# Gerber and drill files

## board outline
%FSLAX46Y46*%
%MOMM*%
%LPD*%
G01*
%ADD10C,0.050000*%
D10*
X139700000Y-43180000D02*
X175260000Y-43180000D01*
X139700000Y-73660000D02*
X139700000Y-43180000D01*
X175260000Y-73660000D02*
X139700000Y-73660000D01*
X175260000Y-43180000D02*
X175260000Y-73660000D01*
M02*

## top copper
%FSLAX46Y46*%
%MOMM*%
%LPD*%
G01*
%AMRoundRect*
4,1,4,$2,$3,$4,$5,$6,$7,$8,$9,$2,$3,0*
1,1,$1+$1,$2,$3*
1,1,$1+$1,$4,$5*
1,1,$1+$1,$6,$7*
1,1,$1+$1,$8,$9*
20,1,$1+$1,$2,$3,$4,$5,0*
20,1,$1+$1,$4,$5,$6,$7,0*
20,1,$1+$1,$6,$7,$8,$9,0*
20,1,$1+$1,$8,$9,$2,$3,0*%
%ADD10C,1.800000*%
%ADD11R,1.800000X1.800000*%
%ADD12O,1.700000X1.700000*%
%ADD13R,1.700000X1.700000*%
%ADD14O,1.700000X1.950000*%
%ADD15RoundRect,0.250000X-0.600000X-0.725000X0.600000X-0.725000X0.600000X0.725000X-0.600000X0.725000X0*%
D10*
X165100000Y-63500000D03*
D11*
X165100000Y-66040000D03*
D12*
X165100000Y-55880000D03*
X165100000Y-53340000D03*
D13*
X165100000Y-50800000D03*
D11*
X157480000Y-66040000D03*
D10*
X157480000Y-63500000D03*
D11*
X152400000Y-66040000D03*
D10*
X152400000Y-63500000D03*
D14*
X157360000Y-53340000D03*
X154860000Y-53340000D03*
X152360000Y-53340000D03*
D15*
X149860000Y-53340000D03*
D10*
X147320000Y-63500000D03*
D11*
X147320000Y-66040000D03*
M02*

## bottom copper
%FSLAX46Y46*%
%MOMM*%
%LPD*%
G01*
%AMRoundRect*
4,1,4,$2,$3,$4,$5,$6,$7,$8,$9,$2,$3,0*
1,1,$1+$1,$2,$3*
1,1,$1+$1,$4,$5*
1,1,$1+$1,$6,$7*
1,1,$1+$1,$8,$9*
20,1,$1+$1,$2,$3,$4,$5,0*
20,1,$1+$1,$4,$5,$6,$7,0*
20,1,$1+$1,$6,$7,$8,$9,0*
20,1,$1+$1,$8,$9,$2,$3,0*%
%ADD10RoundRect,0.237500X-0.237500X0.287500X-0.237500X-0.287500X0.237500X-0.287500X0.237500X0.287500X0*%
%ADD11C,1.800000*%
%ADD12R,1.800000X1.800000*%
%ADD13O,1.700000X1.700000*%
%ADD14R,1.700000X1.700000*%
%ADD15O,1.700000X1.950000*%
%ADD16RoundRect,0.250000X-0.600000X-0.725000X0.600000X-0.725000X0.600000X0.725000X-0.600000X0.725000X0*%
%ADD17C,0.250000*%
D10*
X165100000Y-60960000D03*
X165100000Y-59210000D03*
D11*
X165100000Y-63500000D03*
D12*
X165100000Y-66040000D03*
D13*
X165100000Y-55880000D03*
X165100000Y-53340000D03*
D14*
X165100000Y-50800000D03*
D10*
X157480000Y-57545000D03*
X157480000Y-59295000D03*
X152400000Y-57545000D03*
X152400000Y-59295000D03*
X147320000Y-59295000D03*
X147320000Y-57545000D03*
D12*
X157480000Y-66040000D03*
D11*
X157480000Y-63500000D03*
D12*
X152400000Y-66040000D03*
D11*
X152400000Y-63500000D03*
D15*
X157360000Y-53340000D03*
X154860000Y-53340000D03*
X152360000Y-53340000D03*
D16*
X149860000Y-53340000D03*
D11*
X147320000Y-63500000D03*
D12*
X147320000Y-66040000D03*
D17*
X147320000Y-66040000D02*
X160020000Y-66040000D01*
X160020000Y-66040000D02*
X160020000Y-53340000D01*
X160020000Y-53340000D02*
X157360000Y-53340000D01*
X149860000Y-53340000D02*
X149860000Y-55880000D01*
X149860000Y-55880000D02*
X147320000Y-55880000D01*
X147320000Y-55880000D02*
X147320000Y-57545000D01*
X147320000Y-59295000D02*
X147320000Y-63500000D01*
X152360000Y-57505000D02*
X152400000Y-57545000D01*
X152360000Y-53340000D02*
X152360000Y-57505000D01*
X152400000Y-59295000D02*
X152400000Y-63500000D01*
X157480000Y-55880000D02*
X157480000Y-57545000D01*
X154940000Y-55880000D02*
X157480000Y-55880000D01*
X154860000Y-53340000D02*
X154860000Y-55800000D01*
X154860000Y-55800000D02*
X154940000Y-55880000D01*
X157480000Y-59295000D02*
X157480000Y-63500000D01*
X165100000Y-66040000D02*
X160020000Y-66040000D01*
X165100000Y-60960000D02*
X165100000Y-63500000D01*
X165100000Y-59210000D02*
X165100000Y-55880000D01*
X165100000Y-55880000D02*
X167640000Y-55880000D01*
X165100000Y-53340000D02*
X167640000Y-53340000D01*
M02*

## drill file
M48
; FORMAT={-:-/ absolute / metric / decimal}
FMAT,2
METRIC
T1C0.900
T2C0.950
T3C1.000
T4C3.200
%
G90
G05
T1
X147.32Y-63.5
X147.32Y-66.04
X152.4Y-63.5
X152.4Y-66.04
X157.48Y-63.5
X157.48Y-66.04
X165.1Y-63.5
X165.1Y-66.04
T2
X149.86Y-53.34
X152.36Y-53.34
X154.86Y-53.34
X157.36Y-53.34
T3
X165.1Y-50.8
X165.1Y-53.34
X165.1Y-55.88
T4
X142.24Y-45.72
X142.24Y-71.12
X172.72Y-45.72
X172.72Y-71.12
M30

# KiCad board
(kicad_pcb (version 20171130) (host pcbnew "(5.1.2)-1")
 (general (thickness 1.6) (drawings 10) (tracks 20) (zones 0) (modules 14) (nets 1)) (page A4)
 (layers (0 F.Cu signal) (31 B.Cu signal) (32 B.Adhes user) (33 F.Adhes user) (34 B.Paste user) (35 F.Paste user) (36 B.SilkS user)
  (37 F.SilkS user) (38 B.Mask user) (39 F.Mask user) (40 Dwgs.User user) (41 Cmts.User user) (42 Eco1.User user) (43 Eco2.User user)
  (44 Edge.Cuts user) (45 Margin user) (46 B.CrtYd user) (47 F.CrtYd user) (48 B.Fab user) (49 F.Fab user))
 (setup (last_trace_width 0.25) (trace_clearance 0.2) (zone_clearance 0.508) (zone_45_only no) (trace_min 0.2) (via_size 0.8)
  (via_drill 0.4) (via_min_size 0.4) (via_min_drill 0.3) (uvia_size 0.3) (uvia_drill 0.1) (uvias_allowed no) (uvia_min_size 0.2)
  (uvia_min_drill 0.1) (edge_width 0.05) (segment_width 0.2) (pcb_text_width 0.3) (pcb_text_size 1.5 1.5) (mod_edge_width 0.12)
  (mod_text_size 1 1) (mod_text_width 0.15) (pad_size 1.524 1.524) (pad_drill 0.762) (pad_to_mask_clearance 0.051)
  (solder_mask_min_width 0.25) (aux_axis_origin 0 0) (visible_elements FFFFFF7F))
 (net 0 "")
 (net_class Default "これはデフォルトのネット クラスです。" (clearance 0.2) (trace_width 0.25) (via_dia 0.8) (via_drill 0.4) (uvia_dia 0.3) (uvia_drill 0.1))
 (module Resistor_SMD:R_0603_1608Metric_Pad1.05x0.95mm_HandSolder (layer B.Cu) (at 165.1 60.085 270)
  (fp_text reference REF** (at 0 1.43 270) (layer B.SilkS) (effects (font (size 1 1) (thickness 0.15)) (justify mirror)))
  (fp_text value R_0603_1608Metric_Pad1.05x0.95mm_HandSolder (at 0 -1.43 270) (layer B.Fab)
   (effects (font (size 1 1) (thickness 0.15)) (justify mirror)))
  (pad 2 smd roundrect (at 0.875 0 270) (size 1.05 0.95) (layers B.Cu B.Paste B.Mask) (roundrect_rratio 0.25))
  (pad 1 smd roundrect (at -0.875 0 270) (size 1.05 0.95) (layers B.Cu B.Paste B.Mask) (roundrect_rratio 0.25)))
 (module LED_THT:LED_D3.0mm (layer F.Cu) (at 165.1 66.04 90)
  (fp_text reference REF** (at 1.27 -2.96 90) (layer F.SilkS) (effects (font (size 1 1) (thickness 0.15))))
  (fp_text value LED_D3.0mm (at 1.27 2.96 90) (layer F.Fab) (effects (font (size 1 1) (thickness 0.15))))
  (pad 2 thru_hole circle (at 2.54 0 90) (size 1.8 1.8) (drill 0.9) (layers *.Cu *.Mask))
  (pad 1 thru_hole rect (at 0 0 90) (size 1.8 1.8) (drill 0.9) (layers *.Cu *.Mask)))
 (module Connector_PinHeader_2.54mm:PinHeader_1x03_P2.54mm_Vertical (layer F.Cu) (at 165.1 50.8)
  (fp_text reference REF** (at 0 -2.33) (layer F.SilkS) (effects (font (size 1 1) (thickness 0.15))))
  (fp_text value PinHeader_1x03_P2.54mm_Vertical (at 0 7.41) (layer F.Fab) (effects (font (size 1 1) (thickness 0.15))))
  (pad 3 thru_hole oval (at 0 5.08) (size 1.7 1.7) (drill 1) (layers *.Cu *.Mask))
  (pad 2 thru_hole oval (at 0 2.54) (size 1.7 1.7) (drill 1) (layers *.Cu *.Mask))
  (pad 1 thru_hole rect (at 0 0) (size 1.7 1.7) (drill 1) (layers *.Cu *.Mask)))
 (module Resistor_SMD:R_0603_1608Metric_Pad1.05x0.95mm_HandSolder (layer B.Cu) (at 157.48 58.42 270)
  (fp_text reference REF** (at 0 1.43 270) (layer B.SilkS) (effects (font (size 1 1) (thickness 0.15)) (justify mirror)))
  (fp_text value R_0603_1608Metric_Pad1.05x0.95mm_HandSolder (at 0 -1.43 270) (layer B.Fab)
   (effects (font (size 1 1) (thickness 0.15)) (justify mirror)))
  (pad 1 smd roundrect (at -0.875 0 270) (size 1.05 0.95) (layers B.Cu B.Paste B.Mask) (roundrect_rratio 0.25))
  (pad 2 smd roundrect (at 0.875 0 270) (size 1.05 0.95) (layers B.Cu B.Paste B.Mask) (roundrect_rratio 0.25)))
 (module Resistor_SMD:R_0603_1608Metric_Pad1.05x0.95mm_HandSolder (layer B.Cu) (at 152.4 58.42 270)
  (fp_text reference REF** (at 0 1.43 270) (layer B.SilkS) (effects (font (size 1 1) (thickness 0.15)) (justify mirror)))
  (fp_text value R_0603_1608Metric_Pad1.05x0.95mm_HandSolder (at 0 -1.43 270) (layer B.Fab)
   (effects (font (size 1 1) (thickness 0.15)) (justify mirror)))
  (pad 1 smd roundrect (at -0.875 0 270) (size 1.05 0.95) (layers B.Cu B.Paste B.Mask) (roundrect_rratio 0.25))
  (pad 2 smd roundrect (at 0.875 0 270) (size 1.05 0.95) (layers B.Cu B.Paste B.Mask) (roundrect_rratio 0.25)))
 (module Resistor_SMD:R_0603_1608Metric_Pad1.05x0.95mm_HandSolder (layer B.Cu) (at 147.32 58.42 270)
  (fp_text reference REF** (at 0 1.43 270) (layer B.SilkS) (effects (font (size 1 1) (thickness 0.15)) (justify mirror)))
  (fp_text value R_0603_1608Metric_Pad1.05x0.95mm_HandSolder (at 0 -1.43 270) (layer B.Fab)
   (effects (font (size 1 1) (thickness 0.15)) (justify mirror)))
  (pad 2 smd roundrect (at 0.875 0 270) (size 1.05 0.95) (layers B.Cu B.Paste B.Mask) (roundrect_rratio 0.25))
  (pad 1 smd roundrect (at -0.875 0 270) (size 1.05 0.95) (layers B.Cu B.Paste B.Mask) (roundrect_rratio 0.25)))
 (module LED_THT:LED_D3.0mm (layer F.Cu) (at 157.48 66.04 90)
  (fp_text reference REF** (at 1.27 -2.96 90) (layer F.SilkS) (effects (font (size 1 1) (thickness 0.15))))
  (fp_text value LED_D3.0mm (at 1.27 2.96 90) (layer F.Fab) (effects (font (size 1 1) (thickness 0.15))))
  (pad 1 thru_hole rect (at 0 0 90) (size 1.8 1.8) (drill 0.9) (layers *.Cu *.Mask))
  (pad 2 thru_hole circle (at 2.54 0 90) (size 1.8 1.8) (drill 0.9) (layers *.Cu *.Mask)))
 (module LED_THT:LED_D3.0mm (layer F.Cu) (at 152.4 66.04 90)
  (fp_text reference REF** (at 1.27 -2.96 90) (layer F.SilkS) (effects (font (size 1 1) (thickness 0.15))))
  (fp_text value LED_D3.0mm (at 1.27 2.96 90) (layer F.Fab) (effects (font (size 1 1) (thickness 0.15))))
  (pad 1 thru_hole rect (at 0 0 90) (size 1.8 1.8) (drill 0.9) (layers *.Cu *.Mask))
  (pad 2 thru_hole circle (at 2.54 0 90) (size 1.8 1.8) (drill 0.9) (layers *.Cu *.Mask)))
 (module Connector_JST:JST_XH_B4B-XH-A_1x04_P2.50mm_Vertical (layer F.Cu) (at 149.86 53.34)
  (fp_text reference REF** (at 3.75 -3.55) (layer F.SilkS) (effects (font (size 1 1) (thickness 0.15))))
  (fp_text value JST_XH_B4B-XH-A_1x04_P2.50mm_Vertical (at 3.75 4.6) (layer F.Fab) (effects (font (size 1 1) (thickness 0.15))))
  (pad 4 thru_hole oval (at 7.5 0) (size 1.7 1.95) (drill 0.95) (layers *.Cu *.Mask))
  (pad 3 thru_hole oval (at 5 0) (size 1.7 1.95) (drill 0.95) (layers *.Cu *.Mask))
  (pad 2 thru_hole oval (at 2.5 0) (size 1.7 1.95) (drill 0.95) (layers *.Cu *.Mask))
  (pad 1 thru_hole roundrect (at 0 0) (size 1.7 1.95) (drill 0.95) (layers *.Cu *.Mask) (roundrect_rratio 0.147059)))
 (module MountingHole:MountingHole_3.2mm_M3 (layer F.Cu) (at 172.72 71.12)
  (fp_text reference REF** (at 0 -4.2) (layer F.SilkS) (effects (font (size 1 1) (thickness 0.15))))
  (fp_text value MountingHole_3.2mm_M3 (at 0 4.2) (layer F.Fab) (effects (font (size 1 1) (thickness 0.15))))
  (pad 1 np_thru_hole circle (at 0 0) (size 3.2 3.2) (drill 3.2) (layers *.Cu *.Mask)))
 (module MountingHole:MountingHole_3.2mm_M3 (layer F.Cu) (at 142.24 71.12)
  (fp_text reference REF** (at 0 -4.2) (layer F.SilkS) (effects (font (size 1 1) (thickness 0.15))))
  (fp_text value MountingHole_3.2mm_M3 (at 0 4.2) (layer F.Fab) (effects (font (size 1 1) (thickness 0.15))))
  (pad 1 np_thru_hole circle (at 0 0) (size 3.2 3.2) (drill 3.2) (layers *.Cu *.Mask)))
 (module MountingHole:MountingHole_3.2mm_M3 (layer F.Cu) (at 172.72 45.72)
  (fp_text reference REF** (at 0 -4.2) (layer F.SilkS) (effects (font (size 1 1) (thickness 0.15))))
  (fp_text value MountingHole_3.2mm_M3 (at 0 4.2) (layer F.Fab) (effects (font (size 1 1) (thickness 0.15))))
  (pad 1 np_thru_hole circle (at 0 0) (size 3.2 3.2) (drill 3.2) (layers *.Cu *.Mask)))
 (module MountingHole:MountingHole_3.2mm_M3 (layer F.Cu) (at 142.24 45.72)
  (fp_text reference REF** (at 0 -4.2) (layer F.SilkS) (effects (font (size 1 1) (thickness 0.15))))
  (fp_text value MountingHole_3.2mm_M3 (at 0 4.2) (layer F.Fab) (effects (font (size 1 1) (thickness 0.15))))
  (pad 1 np_thru_hole circle (at 0 0) (size 3.2 3.2) (drill 3.2) (layers *.Cu *.Mask)))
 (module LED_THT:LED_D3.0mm (layer F.Cu) (at 147.32 66.04 90)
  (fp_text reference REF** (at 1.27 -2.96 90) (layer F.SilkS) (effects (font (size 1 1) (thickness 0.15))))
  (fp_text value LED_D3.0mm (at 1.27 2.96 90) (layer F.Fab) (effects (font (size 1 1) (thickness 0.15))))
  (pad 2 thru_hole circle (at 2.54 0 90) (size 1.8 1.8) (drill 0.9) (layers *.Cu *.Mask))
  (pad 1 thru_hole rect (at 0 0 90) (size 1.8 1.8) (drill 0.9) (layers *.Cu *.Mask)))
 (gr_line (start 139.7 43.18) (end 175.26 43.18) (layer Edge.Cuts) (width 0.05))
 (gr_line (start 139.7 73.66) (end 139.7 43.18) (layer Edge.Cuts) (width 0.05))
 (gr_line (start 175.26 73.66) (end 139.7 73.66) (layer Edge.Cuts) (width 0.05))
 (gr_line (start 175.26 43.18) (end 175.26 73.66) (layer Edge.Cuts) (width 0.05))
 (segment (start 147.32 66.04) (end 160.02 66.04) (width 0.25) (layer B.Cu) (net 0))
 (segment (start 160.02 66.04) (end 160.02 53.34) (width 0.25) (layer B.Cu) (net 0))
 (segment (start 160.02 53.34) (end 157.36 53.34) (width 0.25) (layer B.Cu) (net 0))
 (segment (start 149.86 53.34) (end 149.86 55.88) (width 0.25) (layer B.Cu) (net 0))
 (segment (start 149.86 55.88) (end 147.32 55.88) (width 0.25) (layer B.Cu) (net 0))
 (segment (start 147.32 55.88) (end 147.32 57.545) (width 0.25) (layer B.Cu) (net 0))
 (segment (start 147.32 59.295) (end 147.32 63.5) (width 0.25) (layer B.Cu) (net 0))
 (segment (start 152.36 57.505) (end 152.4 57.545) (width 0.25) (layer B.Cu) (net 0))
 (segment (start 152.36 53.34) (end 152.36 57.505) (width 0.25) (layer B.Cu) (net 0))
 (segment (start 152.4 59.295) (end 152.4 63.5) (width 0.25) (layer B.Cu) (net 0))
 (segment (start 157.48 55.88) (end 157.48 57.545) (width 0.25) (layer B.Cu) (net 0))
 (segment (start 154.94 55.88) (end 157.48 55.88) (width 0.25) (layer B.Cu) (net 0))
 (segment (start 154.86 53.34) (end 154.86 55.8) (width 0.25) (layer B.Cu) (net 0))
 (segment (start 154.86 55.8) (end 154.94 55.88) (width 0.25) (layer B.Cu) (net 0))
 (segment (start 157.48 59.295) (end 157.48 63.5) (width 0.25) (layer B.Cu) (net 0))
 (segment (start 165.1 66.04) (end 160.02 66.04) (width 0.25) (layer B.Cu) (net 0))
 (segment (start 165.1 60.96) (end 165.1 63.5) (width 0.25) (layer B.Cu) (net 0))
 (segment (start 165.1 59.21) (end 165.1 55.88) (width 0.25) (layer B.Cu) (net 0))
 (segment (start 165.1 55.88) (end 167.64 55.88) (width 0.25) (layer B.Cu) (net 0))
 (segment (start 165.1 53.34) (end 167.64 53.34) (width 0.25) (layer B.Cu) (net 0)))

